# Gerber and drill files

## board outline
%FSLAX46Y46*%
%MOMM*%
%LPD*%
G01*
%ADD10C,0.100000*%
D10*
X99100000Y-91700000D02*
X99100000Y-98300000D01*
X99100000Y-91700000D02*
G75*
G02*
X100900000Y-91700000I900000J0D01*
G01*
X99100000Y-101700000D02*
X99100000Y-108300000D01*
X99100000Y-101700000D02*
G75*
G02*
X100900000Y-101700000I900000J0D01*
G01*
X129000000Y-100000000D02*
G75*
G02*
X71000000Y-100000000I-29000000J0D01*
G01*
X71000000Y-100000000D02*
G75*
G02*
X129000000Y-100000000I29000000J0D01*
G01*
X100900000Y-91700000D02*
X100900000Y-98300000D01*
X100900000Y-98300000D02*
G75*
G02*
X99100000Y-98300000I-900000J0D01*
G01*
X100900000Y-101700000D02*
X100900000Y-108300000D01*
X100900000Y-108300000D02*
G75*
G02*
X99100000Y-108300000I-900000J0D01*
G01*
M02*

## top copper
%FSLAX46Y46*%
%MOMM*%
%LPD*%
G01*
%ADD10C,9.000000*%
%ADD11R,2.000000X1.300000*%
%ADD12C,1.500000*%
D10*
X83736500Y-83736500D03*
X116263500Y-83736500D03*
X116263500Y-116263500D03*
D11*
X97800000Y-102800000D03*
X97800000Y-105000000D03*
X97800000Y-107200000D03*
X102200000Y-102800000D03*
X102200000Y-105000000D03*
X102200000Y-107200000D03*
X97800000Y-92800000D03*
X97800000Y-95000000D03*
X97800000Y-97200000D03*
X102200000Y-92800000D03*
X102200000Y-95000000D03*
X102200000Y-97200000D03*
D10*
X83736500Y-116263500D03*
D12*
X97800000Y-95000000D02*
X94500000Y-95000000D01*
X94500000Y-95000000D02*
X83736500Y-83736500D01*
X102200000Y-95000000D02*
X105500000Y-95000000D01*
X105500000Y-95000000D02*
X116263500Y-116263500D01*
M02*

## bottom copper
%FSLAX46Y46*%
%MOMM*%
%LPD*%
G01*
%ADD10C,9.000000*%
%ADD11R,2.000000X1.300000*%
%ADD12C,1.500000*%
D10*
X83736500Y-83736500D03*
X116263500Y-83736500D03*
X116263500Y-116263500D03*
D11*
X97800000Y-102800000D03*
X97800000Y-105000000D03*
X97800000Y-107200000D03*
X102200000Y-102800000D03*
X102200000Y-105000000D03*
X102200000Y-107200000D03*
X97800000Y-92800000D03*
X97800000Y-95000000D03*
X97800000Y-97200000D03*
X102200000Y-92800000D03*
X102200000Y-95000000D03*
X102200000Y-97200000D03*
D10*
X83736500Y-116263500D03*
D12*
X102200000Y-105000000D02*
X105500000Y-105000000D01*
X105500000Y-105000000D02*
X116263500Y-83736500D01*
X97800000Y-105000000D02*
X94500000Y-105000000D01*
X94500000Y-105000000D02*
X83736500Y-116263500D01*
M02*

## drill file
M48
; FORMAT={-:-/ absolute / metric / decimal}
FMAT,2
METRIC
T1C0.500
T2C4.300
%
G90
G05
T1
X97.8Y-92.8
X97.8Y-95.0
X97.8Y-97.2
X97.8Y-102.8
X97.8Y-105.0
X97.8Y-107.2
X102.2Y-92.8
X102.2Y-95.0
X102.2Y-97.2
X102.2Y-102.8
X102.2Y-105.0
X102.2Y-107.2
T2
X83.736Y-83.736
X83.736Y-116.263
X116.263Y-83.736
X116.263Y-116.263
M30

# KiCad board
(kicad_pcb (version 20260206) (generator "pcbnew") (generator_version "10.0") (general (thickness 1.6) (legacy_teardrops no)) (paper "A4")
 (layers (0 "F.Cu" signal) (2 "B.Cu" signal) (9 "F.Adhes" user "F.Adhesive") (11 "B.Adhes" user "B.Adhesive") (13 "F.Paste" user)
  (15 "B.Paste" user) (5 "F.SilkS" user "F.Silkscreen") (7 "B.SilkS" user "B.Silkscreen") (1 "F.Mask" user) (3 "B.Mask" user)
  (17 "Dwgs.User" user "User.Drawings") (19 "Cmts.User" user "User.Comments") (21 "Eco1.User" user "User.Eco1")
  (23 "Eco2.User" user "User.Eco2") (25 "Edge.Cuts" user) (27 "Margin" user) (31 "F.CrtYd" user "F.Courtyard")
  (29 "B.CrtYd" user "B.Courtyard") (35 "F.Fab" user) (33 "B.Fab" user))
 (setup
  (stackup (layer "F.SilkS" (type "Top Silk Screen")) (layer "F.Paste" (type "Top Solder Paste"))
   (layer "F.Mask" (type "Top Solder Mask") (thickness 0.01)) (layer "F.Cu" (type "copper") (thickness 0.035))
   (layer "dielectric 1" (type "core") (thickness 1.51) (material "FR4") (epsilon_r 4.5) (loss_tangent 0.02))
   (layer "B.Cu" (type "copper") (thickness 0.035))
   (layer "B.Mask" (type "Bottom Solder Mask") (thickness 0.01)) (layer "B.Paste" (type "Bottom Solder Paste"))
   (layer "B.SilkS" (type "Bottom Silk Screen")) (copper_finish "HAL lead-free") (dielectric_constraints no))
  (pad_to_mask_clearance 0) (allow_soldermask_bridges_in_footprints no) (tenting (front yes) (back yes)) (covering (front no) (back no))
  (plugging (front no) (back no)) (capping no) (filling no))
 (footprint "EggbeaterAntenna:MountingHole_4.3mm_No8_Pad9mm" (layer "F.Cu") (at 83.7365 83.7365)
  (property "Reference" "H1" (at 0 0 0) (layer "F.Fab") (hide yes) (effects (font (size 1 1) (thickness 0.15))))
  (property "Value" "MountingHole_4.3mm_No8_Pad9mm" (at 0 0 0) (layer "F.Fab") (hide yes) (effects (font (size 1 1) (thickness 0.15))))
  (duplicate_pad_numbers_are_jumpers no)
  (pad "1" thru_hole circle (at 0 0) (size 9 9) (drill 4.3) (layers "*.Cu" "*.Mask") (remove_unused_layers no) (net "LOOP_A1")))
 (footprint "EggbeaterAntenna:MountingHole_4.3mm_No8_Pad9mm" (layer "F.Cu") (at 116.2635 83.7365)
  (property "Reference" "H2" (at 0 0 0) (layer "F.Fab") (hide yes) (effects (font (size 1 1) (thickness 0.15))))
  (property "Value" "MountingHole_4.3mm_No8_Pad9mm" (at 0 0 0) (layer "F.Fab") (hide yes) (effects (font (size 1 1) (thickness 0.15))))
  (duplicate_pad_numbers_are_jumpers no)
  (pad "1" thru_hole circle (at 0 0) (size 9 9) (drill 4.3) (layers "*.Cu" "*.Mask") (remove_unused_layers no) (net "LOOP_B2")))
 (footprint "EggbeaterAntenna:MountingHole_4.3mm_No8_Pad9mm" (layer "F.Cu") (at 116.2635 116.2635)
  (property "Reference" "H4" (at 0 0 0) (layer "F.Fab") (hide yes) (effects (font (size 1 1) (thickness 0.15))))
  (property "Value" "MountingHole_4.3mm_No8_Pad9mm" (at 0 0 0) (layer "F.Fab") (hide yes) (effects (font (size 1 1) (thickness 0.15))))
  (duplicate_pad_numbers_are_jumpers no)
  (pad "1" thru_hole circle (at 0 0) (size 9 9) (drill 4.3) (layers "*.Cu" "*.Mask") (remove_unused_layers no) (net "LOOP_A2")))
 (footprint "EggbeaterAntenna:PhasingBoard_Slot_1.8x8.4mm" (layer "F.Cu") (at 100 105)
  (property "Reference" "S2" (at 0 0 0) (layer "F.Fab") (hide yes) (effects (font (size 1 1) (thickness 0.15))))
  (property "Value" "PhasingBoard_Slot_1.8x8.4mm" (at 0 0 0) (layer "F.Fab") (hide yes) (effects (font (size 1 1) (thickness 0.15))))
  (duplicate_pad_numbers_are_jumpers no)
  (pad "1" thru_hole rect (at -2.2 -2.2) (size 2 1.3) (drill 0.5) (layers "*.Cu" "*.Mask") (remove_unused_layers no))
  (pad "2" thru_hole rect (at -2.2 0) (size 2 1.3) (drill 0.5) (layers "*.Cu" "*.Mask") (remove_unused_layers no) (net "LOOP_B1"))
  (pad "3" thru_hole rect (at -2.2 2.2) (size 2 1.3) (drill 0.5) (layers "*.Cu" "*.Mask") (remove_unused_layers no))
  (pad "4" thru_hole rect (at 2.2 -2.2) (size 2 1.3) (drill 0.5) (layers "*.Cu" "*.Mask") (remove_unused_layers no))
  (pad "5" thru_hole rect (at 2.2 0) (size 2 1.3) (drill 0.5) (layers "*.Cu" "*.Mask") (remove_unused_layers no) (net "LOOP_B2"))
  (pad "6" thru_hole rect (at 2.2 2.2) (size 2 1.3) (drill 0.5) (layers "*.Cu" "*.Mask") (remove_unused_layers no)))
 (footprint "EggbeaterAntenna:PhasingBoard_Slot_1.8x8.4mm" (layer "F.Cu") (at 100 95)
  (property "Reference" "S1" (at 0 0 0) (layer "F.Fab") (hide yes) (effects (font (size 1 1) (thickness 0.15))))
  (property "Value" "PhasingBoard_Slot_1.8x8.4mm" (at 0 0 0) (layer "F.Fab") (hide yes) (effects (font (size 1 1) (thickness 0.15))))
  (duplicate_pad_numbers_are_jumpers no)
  (pad "1" thru_hole rect (at -2.2 -2.2) (size 2 1.3) (drill 0.5) (layers "*.Cu" "*.Mask") (remove_unused_layers no))
  (pad "2" thru_hole rect (at -2.2 0) (size 2 1.3) (drill 0.5) (layers "*.Cu" "*.Mask") (remove_unused_layers no) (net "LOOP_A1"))
  (pad "3" thru_hole rect (at -2.2 2.2) (size 2 1.3) (drill 0.5) (layers "*.Cu" "*.Mask") (remove_unused_layers no))
  (pad "4" thru_hole rect (at 2.2 -2.2) (size 2 1.3) (drill 0.5) (layers "*.Cu" "*.Mask") (remove_unused_layers no))
  (pad "5" thru_hole rect (at 2.2 0) (size 2 1.3) (drill 0.5) (layers "*.Cu" "*.Mask") (remove_unused_layers no) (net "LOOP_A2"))
  (pad "6" thru_hole rect (at 2.2 2.2) (size 2 1.3) (drill 0.5) (layers "*.Cu" "*.Mask") (remove_unused_layers no)))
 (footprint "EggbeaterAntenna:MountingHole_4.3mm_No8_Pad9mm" (layer "F.Cu") (at 83.7365 116.2635)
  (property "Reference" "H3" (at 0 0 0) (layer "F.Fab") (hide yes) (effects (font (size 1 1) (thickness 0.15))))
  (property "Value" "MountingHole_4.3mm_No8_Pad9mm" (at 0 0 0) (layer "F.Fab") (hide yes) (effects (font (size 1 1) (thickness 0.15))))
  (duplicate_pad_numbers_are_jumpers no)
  (pad "1" thru_hole circle (at 0 0) (size 9 9) (drill 4.3) (layers "*.Cu" "*.Mask") (remove_unused_layers no) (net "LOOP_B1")))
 (gr_line (start 99.1 91.7) (end 99.1 98.3) (stroke (width 0.1) (type solid)) (layer "Edge.Cuts"))
 (gr_arc (start 99.1 91.7) (mid 100 90.8) (end 100.9 91.7) (stroke (width 0.1) (type solid)) (layer "Edge.Cuts"))
 (gr_line (start 99.1 101.7) (end 99.1 108.3) (stroke (width 0.1) (type solid)) (layer "Edge.Cuts"))
 (gr_arc (start 99.1 101.7) (mid 100 100.8) (end 100.9 101.7) (stroke (width 0.1) (type solid)) (layer "Edge.Cuts"))
 (gr_circle (center 100 100) (end 129 100) (stroke (width 0.1) (type solid)) (fill no) (layer "Edge.Cuts"))
 (gr_line (start 100.9 91.7) (end 100.9 98.3) (stroke (width 0.1) (type solid)) (layer "Edge.Cuts"))
 (gr_arc (start 100.9 98.3) (mid 100 99.2) (end 99.1 98.3) (stroke (width 0.1) (type solid)) (layer "Edge.Cuts"))
 (gr_line (start 100.9 101.7) (end 100.9 108.3) (stroke (width 0.1) (type solid)) (layer "Edge.Cuts"))
 (gr_arc (start 100.9 108.3) (mid 100 109.2) (end 99.1 108.3) (stroke (width 0.1) (type solid)) (layer "Edge.Cuts"))
 (segment (start 97.8 95) (end 94.5 95) (width 1.5) (layer "F.Cu") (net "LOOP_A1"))
 (segment (start 94.5 95) (end 83.7365 83.7365) (width 1.5) (layer "F.Cu") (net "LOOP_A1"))
 (segment (start 102.2 105) (end 105.5 105) (width 1.5) (layer "B.Cu") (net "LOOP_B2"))
 (segment (start 105.5 105) (end 116.2635 83.7365) (width 1.5) (layer "B.Cu") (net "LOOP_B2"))
 (segment (start 102.2 95) (end 105.5 95) (width 1.5) (layer "F.Cu") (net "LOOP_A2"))
 (segment (start 105.5 95) (end 116.2635 116.2635) (width 1.5) (layer "F.Cu") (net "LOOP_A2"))
 (segment (start 97.8 105) (end 94.5 105) (width 1.5) (layer "B.Cu") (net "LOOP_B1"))
 (segment (start 94.5 105) (end 83.7365 116.2635) (width 1.5) (layer "B.Cu") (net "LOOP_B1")))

